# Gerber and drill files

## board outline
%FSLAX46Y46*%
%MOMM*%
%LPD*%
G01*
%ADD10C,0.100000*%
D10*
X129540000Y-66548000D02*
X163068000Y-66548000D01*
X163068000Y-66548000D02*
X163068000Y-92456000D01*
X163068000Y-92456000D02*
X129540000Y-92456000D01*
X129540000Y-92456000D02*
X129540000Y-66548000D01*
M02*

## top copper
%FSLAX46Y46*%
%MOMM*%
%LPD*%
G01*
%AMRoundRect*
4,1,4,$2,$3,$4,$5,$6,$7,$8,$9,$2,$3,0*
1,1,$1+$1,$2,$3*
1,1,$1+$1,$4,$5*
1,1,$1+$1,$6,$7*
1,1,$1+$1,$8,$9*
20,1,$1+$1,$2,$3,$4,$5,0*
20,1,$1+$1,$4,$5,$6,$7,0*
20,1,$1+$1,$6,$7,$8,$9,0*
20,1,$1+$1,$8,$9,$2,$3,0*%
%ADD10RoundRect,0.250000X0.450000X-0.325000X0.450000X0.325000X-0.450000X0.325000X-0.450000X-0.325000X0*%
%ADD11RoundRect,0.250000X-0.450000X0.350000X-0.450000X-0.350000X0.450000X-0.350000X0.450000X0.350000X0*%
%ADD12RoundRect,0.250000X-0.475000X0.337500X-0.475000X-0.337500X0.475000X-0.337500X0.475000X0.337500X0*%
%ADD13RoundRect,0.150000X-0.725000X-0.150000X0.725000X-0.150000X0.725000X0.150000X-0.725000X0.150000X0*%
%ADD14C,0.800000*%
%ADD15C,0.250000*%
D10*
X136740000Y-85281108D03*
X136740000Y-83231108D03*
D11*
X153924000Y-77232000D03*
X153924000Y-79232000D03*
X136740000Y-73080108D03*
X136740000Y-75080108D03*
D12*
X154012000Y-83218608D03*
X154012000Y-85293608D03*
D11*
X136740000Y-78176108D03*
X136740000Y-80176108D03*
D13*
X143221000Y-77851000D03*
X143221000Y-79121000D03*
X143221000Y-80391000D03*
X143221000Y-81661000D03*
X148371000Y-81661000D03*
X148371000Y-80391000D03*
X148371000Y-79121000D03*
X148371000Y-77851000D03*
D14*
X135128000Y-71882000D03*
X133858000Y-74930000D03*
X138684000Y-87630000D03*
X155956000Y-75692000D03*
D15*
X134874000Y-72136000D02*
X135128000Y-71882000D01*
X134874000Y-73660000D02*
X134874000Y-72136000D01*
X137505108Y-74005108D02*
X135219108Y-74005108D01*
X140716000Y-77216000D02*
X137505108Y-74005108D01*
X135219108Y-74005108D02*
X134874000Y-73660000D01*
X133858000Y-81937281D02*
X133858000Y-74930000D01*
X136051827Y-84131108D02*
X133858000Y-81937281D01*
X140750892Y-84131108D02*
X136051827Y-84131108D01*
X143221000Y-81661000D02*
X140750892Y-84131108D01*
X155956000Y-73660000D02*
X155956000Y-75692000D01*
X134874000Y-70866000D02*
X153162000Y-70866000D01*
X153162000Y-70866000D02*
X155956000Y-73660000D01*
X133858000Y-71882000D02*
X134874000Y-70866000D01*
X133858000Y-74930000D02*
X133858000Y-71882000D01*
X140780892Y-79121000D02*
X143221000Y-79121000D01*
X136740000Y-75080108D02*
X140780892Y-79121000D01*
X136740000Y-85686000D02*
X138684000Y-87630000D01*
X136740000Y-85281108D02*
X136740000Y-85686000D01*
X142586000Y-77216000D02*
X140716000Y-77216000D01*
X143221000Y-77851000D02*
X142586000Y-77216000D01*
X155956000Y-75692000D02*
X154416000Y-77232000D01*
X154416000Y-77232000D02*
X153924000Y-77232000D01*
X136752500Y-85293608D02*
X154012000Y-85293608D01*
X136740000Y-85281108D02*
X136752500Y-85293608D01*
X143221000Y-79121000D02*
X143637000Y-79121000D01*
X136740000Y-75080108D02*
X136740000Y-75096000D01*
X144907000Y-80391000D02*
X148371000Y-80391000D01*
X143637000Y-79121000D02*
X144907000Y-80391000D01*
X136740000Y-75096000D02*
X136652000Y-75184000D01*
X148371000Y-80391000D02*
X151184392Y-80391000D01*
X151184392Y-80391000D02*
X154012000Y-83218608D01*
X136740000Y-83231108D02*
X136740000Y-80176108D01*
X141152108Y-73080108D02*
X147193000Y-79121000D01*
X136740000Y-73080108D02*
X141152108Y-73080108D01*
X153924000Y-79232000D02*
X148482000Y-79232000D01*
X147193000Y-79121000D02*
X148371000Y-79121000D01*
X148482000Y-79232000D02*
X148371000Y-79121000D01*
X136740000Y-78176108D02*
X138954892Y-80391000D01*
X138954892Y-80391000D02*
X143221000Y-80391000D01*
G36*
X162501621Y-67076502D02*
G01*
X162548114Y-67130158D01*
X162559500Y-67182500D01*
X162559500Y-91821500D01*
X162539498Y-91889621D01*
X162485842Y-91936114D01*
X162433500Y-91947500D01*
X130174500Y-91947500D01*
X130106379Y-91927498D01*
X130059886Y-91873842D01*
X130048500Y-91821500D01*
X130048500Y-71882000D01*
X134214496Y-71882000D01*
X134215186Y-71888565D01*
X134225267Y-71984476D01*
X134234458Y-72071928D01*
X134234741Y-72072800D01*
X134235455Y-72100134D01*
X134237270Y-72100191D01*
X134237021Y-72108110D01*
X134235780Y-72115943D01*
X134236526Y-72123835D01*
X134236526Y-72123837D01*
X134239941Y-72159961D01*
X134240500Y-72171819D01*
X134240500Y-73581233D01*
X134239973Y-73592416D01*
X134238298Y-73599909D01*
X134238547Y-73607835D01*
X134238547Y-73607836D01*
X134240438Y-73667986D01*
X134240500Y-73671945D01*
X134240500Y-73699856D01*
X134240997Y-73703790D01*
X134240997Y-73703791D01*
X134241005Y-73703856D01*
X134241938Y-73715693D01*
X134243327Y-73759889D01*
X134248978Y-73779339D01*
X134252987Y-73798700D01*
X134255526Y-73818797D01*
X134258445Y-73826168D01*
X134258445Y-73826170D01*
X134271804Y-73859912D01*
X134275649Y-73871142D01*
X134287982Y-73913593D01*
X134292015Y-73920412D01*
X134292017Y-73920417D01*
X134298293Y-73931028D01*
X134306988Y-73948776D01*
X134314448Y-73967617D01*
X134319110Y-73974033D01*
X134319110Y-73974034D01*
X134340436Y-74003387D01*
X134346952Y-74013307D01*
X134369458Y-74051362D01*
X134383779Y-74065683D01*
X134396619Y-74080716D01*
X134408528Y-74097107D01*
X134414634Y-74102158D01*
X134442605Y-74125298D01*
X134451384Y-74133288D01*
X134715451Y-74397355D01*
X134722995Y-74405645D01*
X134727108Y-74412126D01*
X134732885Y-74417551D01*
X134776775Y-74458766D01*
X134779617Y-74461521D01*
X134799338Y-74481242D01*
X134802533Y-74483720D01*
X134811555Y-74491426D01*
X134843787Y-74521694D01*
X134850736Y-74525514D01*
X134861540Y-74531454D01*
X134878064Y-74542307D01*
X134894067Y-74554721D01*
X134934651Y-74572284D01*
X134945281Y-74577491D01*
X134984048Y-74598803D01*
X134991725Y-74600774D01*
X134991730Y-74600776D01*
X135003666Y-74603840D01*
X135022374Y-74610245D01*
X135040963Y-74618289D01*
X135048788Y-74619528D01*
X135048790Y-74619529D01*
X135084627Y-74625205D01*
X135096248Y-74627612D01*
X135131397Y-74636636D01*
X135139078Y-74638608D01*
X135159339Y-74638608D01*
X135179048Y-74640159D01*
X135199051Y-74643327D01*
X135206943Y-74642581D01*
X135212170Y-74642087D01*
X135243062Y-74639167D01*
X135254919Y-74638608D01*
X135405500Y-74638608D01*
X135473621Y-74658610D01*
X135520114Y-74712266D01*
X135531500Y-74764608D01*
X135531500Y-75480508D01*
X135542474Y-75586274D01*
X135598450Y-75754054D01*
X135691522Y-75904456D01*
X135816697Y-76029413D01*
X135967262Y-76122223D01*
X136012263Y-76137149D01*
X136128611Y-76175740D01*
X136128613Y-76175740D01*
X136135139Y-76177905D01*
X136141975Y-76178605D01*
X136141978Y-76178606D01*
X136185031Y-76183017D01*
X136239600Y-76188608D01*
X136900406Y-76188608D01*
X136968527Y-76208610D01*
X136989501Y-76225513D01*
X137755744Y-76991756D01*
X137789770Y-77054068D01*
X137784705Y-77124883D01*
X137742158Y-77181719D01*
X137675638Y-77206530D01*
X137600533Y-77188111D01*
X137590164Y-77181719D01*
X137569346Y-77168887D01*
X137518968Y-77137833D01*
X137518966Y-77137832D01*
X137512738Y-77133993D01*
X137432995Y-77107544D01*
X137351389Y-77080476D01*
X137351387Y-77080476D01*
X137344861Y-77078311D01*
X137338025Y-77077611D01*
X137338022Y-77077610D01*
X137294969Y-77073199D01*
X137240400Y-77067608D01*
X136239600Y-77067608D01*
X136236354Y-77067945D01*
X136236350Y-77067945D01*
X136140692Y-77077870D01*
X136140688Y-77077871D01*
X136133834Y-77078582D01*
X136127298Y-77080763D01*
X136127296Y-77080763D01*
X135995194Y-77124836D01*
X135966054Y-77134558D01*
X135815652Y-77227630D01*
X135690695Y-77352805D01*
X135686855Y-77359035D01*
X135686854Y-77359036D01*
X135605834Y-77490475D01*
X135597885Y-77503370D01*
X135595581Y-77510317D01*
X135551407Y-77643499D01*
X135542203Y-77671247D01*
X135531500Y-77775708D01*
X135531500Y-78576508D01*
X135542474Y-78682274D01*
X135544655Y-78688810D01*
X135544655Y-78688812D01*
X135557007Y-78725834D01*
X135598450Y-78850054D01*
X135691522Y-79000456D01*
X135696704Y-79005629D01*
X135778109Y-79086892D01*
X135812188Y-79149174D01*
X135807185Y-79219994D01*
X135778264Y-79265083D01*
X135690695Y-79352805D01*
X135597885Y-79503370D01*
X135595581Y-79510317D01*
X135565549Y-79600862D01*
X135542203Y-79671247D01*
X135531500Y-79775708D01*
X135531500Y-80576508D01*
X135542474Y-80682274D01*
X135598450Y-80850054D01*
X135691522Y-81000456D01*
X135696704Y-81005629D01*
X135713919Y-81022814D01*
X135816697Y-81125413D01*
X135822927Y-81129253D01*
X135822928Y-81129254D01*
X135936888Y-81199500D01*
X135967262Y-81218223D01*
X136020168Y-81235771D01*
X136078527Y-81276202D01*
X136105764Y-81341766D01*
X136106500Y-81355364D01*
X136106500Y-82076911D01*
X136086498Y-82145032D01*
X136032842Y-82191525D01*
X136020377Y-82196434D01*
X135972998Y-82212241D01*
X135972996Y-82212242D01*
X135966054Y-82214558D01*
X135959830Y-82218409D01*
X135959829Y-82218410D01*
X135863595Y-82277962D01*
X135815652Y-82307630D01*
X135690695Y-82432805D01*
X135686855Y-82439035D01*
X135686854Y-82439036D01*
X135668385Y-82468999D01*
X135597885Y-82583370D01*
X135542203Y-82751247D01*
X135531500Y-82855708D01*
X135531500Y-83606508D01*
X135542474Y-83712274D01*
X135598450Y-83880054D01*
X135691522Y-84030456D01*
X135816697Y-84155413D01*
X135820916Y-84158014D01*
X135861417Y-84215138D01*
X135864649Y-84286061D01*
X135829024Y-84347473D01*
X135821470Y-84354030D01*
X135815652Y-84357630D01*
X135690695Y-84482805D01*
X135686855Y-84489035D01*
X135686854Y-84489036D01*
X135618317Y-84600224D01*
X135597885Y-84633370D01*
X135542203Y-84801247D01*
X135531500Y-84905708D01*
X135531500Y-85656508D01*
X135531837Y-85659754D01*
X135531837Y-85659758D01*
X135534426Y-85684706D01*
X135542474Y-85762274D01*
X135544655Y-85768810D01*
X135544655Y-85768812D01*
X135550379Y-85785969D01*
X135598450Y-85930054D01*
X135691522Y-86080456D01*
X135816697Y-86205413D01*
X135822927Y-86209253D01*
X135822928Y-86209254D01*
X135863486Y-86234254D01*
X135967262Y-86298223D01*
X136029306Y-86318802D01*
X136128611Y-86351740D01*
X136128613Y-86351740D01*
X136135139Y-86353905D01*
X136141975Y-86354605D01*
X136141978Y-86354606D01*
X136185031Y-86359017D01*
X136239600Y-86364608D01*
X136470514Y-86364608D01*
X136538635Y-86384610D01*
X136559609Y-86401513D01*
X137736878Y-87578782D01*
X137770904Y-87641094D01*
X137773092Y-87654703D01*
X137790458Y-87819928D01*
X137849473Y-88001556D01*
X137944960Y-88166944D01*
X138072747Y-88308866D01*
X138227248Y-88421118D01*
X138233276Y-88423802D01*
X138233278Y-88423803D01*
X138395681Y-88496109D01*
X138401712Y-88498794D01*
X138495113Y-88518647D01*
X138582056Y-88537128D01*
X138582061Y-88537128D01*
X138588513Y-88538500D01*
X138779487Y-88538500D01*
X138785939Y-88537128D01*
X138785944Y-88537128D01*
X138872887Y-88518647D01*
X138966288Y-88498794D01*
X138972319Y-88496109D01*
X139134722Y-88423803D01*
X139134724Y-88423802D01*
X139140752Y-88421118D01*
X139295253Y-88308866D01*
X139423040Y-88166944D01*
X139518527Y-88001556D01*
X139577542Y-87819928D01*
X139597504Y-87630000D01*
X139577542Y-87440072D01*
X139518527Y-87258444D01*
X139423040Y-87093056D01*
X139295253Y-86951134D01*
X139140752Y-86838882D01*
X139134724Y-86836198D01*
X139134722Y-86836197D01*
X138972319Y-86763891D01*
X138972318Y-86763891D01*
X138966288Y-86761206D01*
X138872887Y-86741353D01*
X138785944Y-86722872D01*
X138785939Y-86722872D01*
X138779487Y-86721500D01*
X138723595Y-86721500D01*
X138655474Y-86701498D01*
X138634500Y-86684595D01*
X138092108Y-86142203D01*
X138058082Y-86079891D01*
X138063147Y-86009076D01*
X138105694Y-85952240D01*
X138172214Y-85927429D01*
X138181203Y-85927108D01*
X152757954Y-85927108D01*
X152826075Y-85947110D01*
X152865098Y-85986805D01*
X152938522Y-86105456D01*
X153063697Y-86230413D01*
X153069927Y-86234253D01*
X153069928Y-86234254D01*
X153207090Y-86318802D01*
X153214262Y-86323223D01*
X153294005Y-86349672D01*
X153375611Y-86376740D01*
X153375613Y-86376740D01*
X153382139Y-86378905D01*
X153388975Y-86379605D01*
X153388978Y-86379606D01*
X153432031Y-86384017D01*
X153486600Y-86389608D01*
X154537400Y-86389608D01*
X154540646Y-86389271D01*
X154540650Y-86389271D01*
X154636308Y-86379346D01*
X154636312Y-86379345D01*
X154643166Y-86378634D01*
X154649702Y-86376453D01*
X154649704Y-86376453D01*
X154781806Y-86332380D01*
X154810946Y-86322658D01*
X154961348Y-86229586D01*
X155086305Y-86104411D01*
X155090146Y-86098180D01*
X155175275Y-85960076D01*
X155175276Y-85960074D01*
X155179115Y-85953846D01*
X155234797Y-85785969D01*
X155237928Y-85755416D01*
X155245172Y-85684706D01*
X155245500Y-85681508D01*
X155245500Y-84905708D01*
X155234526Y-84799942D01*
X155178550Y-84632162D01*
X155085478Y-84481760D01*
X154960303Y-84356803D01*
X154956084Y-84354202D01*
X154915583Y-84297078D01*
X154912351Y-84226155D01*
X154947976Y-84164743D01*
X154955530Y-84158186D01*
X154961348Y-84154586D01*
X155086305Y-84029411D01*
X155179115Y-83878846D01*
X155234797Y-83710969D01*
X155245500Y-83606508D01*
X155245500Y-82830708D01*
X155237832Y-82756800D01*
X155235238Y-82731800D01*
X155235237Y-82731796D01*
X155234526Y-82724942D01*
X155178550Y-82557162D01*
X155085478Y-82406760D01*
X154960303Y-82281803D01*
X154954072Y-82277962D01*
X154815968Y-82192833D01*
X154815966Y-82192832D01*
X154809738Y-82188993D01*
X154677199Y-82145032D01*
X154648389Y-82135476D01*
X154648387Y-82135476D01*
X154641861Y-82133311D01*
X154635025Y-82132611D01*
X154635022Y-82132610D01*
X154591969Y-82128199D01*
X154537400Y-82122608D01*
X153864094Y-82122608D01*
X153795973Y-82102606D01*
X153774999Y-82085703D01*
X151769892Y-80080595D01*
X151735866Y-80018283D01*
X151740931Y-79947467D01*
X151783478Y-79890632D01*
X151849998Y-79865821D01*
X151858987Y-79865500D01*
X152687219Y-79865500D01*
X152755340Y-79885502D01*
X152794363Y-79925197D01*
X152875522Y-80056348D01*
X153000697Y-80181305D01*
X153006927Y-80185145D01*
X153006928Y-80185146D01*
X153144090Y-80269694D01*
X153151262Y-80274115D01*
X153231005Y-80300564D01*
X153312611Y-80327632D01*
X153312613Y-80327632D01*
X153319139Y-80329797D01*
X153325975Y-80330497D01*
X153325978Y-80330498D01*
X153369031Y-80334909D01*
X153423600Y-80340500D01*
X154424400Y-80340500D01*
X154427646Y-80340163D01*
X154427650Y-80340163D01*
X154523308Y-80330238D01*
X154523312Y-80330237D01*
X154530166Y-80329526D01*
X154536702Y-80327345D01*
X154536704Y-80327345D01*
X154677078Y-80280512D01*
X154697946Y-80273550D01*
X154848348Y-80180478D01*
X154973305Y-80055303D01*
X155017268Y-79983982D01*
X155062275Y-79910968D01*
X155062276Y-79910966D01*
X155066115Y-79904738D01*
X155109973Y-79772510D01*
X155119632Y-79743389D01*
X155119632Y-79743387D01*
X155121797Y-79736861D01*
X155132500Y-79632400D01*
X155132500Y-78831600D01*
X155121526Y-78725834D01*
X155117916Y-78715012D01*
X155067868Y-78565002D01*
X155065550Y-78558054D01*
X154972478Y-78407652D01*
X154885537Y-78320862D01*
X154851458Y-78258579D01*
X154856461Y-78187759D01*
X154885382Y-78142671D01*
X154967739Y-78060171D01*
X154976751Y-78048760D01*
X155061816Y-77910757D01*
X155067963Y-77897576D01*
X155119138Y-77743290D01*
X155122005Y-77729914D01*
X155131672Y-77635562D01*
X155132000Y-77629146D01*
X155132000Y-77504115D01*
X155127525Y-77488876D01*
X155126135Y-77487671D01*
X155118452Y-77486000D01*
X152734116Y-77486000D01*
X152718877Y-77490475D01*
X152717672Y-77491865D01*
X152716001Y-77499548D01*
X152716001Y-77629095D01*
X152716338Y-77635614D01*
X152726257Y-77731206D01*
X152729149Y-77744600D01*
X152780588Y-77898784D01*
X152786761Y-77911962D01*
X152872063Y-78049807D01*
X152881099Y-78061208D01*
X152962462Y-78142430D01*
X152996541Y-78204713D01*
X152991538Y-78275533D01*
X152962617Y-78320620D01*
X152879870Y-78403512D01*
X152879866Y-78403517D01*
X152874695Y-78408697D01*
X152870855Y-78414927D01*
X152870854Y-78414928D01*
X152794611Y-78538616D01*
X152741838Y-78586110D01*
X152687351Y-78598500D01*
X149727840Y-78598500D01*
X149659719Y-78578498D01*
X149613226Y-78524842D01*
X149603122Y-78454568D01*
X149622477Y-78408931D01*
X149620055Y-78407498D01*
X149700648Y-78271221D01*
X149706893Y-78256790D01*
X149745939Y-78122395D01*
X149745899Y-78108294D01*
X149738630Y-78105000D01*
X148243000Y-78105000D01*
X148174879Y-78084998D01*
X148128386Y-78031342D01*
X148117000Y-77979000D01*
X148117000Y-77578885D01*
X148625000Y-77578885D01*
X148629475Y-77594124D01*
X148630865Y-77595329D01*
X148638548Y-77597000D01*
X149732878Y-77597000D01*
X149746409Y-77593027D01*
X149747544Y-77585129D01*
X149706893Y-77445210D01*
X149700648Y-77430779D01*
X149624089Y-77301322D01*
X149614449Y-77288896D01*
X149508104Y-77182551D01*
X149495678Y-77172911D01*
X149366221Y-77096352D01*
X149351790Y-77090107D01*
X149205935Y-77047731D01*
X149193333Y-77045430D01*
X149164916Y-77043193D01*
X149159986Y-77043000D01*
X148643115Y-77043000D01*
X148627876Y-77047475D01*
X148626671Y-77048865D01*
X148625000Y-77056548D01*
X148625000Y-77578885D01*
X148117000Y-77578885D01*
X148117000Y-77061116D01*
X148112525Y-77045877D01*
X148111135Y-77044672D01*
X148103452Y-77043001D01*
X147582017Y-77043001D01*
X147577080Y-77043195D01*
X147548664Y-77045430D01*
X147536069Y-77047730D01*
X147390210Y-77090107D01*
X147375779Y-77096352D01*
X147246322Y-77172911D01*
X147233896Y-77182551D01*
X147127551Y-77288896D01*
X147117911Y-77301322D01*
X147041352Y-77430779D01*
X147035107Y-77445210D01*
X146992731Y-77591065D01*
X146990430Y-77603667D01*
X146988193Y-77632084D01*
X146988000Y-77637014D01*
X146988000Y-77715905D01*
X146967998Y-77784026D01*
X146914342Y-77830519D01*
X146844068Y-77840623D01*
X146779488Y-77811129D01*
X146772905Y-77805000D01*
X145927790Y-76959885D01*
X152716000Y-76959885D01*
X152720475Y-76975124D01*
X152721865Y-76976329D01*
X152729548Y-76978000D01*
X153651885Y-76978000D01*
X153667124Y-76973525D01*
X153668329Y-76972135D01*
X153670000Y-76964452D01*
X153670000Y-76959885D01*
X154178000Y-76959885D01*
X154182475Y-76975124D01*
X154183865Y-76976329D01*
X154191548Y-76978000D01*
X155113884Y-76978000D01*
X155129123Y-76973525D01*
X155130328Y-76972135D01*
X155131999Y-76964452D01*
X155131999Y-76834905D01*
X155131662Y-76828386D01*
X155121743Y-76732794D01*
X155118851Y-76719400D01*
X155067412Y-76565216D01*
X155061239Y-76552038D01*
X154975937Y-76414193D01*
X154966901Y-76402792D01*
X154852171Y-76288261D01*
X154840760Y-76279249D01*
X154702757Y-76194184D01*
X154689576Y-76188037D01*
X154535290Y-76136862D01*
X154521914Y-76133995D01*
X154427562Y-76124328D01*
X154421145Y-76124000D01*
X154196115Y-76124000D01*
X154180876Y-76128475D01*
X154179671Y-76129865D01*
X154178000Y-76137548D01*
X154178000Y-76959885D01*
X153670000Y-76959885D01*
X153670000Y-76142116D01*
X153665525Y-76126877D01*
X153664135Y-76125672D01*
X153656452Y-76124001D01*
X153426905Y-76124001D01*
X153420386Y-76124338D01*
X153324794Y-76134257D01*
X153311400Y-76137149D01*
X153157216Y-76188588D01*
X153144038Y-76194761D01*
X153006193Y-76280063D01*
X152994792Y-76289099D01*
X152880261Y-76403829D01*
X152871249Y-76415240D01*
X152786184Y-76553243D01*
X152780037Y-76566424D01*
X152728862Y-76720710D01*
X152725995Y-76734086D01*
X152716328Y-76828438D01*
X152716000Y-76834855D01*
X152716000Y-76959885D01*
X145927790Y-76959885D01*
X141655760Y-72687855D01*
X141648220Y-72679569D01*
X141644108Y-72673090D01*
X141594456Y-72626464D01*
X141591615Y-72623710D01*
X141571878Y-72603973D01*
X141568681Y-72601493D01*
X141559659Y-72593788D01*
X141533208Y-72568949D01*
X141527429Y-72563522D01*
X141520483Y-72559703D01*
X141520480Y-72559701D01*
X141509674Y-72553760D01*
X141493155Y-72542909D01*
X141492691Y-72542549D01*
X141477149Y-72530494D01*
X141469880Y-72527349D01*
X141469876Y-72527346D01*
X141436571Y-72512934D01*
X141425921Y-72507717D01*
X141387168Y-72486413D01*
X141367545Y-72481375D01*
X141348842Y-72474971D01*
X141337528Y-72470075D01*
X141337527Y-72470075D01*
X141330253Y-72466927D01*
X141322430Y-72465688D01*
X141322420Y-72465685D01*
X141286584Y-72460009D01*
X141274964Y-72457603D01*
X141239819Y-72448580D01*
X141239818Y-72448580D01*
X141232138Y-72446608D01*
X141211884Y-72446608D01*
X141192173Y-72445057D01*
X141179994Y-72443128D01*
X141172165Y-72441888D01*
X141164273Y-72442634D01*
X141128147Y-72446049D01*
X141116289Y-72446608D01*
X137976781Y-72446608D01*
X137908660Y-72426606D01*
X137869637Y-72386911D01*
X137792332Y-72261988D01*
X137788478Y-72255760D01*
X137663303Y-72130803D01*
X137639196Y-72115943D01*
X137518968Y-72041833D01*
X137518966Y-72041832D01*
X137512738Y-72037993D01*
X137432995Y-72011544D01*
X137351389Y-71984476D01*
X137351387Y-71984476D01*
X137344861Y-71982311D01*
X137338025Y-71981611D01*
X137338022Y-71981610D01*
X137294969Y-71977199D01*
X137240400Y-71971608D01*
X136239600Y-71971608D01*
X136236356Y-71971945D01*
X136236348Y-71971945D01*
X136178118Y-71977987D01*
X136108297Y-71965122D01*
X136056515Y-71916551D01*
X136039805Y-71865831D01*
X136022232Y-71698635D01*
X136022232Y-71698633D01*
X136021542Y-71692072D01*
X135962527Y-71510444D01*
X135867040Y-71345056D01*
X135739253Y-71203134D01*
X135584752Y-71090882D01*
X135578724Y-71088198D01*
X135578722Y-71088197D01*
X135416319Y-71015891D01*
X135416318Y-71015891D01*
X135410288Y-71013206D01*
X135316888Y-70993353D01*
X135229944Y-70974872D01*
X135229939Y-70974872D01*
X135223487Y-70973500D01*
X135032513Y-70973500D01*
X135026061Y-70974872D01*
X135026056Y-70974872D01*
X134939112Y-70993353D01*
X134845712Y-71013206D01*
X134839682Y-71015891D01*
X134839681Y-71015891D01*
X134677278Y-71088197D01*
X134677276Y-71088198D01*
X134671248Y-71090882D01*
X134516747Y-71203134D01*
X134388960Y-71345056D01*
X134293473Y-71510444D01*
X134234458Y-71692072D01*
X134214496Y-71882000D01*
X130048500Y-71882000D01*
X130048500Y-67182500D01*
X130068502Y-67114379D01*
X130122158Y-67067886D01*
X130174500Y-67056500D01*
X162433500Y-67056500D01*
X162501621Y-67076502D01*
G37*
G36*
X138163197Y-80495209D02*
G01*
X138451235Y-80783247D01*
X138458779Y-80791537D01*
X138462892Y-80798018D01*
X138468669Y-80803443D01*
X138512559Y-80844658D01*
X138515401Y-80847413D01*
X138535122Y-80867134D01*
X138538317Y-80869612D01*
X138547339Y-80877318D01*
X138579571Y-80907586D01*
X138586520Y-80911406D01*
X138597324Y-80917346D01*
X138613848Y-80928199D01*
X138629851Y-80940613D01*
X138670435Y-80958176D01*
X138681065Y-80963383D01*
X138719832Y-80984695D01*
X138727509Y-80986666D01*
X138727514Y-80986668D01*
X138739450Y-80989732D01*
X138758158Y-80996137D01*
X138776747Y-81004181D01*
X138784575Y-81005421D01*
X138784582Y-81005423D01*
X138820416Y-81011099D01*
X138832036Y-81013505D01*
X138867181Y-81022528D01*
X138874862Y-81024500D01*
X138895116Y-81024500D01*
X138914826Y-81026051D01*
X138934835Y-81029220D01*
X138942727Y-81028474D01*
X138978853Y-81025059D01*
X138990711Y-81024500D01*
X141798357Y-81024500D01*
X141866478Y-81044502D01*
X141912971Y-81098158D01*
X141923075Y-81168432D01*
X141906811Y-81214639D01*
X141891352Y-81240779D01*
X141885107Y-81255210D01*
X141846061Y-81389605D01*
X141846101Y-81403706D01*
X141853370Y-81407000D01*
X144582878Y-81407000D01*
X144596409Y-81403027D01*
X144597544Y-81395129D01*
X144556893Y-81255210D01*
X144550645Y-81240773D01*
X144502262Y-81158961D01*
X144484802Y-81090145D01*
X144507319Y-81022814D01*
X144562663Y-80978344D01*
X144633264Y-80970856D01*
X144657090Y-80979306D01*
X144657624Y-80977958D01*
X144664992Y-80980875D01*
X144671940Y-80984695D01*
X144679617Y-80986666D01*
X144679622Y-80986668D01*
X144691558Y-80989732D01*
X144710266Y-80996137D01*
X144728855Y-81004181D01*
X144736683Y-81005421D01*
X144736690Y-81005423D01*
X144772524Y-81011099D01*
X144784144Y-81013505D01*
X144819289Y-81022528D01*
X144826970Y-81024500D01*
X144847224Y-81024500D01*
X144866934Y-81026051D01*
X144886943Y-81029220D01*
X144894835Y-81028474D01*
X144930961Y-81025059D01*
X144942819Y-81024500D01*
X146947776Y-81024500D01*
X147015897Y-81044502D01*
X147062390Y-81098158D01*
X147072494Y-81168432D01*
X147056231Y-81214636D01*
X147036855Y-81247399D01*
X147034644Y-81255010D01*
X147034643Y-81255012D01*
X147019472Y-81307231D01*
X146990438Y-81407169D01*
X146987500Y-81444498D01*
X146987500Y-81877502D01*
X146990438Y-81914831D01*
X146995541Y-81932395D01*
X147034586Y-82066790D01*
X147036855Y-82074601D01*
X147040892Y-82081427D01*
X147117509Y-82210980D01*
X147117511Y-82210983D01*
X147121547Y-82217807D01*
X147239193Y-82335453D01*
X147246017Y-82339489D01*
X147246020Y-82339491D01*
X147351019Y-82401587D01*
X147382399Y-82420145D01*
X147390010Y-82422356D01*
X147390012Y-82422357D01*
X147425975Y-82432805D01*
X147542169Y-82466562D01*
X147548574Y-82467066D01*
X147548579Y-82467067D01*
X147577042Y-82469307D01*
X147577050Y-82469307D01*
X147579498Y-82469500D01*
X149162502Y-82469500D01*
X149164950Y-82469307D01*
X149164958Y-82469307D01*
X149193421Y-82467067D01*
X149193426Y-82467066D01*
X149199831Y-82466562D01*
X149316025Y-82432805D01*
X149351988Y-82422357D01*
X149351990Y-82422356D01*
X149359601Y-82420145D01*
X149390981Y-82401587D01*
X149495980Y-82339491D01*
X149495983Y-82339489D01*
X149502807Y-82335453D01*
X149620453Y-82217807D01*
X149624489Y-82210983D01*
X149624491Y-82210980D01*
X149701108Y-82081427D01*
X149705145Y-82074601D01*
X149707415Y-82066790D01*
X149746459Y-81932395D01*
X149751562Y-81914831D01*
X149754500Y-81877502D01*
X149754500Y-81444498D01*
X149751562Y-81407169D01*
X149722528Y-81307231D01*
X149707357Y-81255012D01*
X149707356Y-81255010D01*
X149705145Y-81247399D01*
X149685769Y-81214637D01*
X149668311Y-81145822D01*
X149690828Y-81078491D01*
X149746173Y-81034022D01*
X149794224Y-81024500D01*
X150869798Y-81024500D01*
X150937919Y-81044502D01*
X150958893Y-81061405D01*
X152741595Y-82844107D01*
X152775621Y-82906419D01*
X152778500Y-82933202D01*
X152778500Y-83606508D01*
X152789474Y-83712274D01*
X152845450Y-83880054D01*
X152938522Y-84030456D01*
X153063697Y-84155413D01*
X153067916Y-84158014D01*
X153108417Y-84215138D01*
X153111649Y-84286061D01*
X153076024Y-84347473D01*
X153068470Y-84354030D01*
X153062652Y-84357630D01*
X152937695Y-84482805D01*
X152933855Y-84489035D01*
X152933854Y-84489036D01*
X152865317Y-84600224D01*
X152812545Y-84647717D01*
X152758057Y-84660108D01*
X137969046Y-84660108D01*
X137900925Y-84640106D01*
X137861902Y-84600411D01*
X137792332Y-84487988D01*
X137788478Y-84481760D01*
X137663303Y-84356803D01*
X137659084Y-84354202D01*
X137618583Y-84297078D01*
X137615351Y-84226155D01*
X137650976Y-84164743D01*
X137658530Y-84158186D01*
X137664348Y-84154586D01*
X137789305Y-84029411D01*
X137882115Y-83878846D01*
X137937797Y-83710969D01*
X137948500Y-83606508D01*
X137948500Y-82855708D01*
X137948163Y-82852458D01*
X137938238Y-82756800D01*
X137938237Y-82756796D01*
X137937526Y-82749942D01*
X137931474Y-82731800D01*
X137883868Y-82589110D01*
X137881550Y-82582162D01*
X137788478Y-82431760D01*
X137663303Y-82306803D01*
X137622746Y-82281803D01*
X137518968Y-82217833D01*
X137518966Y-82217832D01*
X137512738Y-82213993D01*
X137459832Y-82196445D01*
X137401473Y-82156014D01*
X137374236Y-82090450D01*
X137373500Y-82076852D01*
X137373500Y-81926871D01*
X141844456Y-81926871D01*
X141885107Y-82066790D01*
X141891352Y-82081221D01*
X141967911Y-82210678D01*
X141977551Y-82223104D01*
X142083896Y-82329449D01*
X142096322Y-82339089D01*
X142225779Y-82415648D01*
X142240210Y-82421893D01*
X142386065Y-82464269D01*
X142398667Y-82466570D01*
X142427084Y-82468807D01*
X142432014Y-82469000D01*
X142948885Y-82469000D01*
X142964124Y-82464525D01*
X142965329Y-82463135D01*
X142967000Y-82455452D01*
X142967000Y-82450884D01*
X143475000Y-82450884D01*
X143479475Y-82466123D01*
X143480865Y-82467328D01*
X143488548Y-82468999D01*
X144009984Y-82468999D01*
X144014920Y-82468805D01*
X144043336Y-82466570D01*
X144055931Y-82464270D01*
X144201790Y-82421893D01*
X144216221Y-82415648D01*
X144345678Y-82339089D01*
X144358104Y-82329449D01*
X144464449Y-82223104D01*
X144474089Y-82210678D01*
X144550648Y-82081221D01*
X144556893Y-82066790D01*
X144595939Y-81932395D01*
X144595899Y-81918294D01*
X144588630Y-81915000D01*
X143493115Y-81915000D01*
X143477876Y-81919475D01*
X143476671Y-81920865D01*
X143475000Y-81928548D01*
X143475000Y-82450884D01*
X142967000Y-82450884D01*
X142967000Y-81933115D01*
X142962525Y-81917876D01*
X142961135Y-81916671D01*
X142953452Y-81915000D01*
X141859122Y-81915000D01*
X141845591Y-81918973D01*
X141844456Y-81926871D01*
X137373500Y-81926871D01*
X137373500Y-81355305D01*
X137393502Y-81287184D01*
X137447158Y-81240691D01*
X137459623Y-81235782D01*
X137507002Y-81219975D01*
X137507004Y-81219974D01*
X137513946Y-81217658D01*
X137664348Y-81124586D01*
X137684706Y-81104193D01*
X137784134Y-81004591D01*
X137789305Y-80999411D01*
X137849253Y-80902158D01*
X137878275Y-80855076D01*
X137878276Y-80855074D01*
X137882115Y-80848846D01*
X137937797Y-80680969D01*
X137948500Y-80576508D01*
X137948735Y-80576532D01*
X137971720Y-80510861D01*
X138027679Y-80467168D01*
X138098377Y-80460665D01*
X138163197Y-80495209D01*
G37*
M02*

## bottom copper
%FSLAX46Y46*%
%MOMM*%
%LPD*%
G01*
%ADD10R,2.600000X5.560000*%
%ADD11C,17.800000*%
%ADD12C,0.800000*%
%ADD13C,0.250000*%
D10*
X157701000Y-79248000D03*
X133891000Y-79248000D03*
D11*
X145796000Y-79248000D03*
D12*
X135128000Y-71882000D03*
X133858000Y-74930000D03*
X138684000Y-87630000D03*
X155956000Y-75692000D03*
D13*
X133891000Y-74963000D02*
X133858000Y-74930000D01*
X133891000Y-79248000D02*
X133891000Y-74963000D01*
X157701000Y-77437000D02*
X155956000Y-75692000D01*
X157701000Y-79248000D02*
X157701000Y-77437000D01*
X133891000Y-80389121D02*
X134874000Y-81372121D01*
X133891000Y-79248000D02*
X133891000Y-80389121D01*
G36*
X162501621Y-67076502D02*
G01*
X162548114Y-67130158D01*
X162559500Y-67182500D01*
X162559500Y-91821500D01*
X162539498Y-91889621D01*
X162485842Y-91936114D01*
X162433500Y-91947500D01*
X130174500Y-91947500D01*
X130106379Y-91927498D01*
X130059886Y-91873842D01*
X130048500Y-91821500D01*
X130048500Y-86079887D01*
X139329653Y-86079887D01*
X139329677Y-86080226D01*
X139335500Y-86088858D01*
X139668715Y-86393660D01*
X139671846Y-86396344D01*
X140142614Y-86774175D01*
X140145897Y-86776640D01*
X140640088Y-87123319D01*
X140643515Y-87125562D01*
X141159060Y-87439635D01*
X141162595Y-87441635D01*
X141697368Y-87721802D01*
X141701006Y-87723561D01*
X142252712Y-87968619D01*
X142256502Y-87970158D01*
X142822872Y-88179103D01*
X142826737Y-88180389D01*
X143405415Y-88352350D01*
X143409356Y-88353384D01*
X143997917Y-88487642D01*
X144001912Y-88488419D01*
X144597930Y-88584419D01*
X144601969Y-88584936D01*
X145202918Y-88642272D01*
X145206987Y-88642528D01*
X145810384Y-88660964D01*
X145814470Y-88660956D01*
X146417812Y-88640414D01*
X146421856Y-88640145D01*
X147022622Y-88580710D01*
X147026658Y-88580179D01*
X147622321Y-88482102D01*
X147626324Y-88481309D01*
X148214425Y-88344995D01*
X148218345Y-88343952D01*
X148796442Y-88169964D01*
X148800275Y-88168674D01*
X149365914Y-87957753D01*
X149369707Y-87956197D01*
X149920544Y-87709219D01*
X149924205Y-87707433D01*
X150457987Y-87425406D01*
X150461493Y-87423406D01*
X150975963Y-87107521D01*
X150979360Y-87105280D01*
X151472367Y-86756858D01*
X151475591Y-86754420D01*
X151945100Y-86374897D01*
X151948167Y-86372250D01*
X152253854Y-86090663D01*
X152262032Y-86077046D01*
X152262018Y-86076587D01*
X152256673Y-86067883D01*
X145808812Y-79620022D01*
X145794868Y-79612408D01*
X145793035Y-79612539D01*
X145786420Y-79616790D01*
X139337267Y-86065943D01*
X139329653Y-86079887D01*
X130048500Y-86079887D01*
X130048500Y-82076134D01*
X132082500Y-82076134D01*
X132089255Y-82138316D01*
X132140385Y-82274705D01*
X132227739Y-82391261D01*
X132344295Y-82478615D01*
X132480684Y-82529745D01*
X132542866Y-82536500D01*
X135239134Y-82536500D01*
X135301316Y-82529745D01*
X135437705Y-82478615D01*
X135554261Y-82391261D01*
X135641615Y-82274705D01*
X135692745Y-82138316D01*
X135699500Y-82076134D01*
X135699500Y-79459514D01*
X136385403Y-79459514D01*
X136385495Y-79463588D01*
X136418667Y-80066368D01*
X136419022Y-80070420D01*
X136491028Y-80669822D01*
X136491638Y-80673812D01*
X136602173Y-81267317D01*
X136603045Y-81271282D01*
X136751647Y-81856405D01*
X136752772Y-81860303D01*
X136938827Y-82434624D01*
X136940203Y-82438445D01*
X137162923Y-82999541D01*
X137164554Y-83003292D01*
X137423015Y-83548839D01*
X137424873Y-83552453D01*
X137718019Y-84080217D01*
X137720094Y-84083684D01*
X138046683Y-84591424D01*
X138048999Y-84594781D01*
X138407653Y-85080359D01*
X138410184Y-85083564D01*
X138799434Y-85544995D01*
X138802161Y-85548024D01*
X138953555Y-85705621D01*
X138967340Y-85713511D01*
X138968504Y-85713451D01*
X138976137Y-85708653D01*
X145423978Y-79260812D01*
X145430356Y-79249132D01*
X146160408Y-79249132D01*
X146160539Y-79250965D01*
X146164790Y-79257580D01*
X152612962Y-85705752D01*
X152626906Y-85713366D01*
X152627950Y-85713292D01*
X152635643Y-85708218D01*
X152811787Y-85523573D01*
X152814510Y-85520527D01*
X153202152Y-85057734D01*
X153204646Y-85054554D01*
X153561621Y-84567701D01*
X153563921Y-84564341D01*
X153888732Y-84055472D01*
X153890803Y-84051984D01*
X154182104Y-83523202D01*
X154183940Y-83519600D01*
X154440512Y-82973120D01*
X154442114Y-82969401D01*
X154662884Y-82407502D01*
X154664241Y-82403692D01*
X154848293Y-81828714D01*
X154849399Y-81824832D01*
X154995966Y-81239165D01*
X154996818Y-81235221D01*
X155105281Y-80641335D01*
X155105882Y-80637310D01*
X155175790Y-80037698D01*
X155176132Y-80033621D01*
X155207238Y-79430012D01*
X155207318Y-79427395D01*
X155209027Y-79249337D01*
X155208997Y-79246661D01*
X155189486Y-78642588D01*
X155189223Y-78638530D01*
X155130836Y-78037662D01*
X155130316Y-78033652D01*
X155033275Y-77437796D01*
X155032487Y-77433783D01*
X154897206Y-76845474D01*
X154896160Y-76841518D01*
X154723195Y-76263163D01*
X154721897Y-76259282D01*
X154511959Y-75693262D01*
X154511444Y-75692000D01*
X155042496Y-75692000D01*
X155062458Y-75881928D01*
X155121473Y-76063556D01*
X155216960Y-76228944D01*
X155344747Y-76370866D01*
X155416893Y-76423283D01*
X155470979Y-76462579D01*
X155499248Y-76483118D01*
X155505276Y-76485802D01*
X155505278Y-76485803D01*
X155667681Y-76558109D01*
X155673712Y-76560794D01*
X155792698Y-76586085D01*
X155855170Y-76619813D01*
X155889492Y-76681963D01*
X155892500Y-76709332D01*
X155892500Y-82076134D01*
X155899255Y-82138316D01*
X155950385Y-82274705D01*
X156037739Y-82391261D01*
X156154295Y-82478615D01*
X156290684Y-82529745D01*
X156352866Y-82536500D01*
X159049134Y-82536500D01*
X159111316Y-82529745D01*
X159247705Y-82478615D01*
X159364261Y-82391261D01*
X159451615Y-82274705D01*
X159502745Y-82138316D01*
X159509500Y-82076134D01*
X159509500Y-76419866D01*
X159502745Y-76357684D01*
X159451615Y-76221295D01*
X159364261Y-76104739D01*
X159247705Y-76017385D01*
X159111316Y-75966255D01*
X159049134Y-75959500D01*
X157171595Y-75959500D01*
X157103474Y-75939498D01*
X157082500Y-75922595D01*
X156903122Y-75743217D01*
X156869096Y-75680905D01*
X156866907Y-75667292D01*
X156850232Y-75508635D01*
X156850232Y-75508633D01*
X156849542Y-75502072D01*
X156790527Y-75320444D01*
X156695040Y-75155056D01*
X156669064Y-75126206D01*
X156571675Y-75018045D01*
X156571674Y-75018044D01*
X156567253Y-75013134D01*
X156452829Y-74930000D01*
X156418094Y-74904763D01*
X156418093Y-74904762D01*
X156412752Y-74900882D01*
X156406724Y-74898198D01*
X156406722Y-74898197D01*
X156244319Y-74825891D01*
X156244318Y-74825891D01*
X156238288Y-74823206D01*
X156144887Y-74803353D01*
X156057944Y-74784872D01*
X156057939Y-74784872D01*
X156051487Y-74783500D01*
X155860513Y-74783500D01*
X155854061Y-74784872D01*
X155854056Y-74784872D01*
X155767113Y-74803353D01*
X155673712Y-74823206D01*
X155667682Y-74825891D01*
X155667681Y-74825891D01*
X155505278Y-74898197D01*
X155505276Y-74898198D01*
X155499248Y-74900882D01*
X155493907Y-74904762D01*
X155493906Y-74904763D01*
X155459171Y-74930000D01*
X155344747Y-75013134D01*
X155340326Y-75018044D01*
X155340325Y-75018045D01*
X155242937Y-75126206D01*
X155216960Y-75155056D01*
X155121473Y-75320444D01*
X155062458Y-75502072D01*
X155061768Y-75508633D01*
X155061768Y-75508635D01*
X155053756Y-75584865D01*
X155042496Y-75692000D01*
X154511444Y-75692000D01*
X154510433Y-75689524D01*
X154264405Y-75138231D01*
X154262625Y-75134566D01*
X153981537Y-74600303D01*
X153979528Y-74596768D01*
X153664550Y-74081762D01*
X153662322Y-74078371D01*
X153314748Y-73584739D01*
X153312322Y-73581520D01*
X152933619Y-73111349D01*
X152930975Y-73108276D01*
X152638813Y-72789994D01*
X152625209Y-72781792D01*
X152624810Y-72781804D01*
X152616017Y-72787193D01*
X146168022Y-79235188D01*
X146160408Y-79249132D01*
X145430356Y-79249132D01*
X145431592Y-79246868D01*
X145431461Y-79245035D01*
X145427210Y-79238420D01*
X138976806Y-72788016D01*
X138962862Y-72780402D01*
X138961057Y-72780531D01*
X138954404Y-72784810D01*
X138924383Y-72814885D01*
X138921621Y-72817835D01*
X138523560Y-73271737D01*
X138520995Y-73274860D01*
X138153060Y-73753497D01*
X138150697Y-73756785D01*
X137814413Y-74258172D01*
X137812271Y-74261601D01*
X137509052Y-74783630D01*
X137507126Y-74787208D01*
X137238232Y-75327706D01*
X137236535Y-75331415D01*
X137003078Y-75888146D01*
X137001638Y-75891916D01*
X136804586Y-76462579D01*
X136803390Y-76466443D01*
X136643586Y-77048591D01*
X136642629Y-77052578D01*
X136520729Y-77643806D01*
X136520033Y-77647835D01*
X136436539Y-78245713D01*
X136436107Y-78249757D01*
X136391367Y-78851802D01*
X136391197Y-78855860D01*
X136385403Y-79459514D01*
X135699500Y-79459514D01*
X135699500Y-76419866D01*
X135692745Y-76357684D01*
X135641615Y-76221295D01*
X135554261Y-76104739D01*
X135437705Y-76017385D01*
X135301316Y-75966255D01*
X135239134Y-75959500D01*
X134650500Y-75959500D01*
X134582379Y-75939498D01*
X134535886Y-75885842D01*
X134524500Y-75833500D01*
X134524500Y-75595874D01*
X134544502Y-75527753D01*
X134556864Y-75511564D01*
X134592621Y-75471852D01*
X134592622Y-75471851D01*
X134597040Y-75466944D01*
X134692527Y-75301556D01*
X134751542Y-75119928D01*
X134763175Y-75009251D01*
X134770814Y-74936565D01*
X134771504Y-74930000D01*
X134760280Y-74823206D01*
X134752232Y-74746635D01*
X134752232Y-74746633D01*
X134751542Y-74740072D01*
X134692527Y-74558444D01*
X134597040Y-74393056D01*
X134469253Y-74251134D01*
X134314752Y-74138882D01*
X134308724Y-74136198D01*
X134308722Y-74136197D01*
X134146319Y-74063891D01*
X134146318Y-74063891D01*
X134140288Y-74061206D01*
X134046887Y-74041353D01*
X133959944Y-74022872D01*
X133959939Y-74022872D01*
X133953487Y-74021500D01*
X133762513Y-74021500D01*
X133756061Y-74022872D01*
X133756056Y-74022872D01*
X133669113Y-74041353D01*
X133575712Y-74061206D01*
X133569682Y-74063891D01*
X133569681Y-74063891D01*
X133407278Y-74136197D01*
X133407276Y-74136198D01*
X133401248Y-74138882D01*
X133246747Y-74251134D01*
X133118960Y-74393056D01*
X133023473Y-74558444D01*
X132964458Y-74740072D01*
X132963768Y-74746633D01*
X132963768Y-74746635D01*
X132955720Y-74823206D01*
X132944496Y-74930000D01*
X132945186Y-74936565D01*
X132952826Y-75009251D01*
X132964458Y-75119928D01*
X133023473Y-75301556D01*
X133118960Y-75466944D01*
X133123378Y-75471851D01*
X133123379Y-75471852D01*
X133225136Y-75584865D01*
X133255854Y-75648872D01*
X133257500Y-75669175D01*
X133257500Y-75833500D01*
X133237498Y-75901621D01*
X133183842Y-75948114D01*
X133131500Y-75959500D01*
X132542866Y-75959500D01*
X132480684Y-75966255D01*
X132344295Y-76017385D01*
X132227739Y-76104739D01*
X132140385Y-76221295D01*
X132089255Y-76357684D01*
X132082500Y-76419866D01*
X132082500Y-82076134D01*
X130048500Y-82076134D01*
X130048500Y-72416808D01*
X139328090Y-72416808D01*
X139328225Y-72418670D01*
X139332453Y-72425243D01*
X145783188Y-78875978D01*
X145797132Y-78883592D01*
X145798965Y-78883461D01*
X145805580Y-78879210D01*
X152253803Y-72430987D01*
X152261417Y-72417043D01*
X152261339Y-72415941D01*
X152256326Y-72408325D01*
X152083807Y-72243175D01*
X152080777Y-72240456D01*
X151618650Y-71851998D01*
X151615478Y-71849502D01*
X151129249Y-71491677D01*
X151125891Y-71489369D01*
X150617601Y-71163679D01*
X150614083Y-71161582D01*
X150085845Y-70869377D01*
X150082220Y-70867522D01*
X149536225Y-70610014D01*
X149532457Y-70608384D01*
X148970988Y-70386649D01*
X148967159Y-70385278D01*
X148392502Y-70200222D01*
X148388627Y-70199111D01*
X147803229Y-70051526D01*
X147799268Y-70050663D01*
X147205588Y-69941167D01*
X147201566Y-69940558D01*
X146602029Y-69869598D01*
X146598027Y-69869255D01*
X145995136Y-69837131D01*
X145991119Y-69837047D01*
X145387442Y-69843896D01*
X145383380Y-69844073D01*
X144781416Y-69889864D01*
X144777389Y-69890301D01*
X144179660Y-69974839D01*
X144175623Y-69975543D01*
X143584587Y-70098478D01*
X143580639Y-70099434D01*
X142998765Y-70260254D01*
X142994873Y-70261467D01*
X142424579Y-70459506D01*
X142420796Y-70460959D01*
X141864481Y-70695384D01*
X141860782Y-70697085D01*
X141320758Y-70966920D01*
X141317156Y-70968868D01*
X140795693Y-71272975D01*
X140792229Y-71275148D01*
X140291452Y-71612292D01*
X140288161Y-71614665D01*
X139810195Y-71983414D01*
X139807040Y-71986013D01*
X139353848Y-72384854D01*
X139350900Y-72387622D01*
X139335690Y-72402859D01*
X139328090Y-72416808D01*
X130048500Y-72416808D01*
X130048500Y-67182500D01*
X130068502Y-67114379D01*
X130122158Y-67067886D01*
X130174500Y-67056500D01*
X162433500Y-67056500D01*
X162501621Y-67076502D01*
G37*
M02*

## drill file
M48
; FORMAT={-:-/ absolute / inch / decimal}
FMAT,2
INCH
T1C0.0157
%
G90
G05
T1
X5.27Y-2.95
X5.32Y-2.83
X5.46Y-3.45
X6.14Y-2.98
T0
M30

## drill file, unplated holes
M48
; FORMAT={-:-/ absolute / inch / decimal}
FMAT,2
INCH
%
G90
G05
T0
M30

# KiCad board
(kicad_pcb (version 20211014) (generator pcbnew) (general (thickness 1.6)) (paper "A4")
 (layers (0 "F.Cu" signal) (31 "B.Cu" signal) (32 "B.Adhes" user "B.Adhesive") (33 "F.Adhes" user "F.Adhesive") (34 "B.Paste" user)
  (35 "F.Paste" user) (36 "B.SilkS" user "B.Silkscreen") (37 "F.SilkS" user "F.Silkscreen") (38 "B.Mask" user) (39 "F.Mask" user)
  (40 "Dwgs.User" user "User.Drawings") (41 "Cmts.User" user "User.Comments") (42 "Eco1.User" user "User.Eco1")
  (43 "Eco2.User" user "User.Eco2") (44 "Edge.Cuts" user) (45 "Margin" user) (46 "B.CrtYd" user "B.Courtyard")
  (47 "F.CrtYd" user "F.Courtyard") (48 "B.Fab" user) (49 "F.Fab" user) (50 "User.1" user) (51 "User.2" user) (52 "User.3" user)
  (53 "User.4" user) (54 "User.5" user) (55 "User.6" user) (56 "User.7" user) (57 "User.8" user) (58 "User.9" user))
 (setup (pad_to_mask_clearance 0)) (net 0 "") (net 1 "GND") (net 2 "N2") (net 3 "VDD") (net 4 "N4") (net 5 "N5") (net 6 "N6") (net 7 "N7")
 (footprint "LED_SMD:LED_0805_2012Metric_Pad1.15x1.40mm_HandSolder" (layer "F.Cu") (at 136.74 84.256108 90)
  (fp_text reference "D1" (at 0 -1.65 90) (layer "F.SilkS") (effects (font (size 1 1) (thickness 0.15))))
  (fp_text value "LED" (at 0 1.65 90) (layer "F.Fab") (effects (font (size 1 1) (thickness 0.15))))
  (pad "1" smd roundrect (at -1.025 0 90) (size 1.15 1.4) (layers "F.Cu" "F.Paste" "F.Mask") (roundrect_rratio 0.2173913043) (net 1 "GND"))
  (pad "2" smd roundrect (at 1.025 0 90) (size 1.15 1.4) (layers "F.Cu" "F.Paste" "F.Mask") (roundrect_rratio 0.2173913043) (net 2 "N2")))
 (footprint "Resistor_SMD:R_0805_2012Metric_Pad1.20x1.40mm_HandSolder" (layer "F.Cu") (at 153.924 78.232 -90)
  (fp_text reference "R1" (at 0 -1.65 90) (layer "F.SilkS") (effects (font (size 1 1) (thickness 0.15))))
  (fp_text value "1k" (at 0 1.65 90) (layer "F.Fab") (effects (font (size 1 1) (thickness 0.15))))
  (pad "1" smd roundrect (at -1 0 270) (size 1.2 1.4) (layers "F.Cu" "F.Paste" "F.Mask") (roundrect_rratio 0.2083333333) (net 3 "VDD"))
  (pad "2" smd roundrect (at 1 0 270) (size 1.2 1.4) (layers "F.Cu" "F.Paste" "F.Mask") (roundrect_rratio 0.2083333333) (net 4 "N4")))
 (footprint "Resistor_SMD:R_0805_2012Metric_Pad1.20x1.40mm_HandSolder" (layer "F.Cu") (at 136.74 74.080108 -90)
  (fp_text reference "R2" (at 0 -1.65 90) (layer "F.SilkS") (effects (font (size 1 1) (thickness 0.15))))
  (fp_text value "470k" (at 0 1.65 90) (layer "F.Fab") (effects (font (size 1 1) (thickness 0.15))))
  (pad "1" smd roundrect (at -1 0 270) (size 1.2 1.4) (layers "F.Cu" "F.Paste" "F.Mask") (roundrect_rratio 0.2083333333) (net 4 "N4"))
  (pad "2" smd roundrect (at 1 0 270) (size 1.2 1.4) (layers "F.Cu" "F.Paste" "F.Mask") (roundrect_rratio 0.2083333333) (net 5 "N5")))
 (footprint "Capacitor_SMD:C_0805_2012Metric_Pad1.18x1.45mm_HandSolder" (layer "F.Cu") (at 154.012 84.256108 -90)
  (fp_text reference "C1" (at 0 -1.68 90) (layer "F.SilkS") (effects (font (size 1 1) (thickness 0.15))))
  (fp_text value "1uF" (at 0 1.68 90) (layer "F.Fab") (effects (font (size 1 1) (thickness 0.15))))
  (pad "1" smd roundrect (at -1.0375 0 270) (size 1.175 1.45) (layers "F.Cu" "F.Paste" "F.Mask") (roundrect_rratio 0.2127659574)
   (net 5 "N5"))
  (pad "2" smd roundrect (at 1.0375 0 270) (size 1.175 1.45) (layers "F.Cu" "F.Paste" "F.Mask") (roundrect_rratio 0.2127659574)
   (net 1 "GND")))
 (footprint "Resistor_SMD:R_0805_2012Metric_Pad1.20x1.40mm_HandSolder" (layer "F.Cu") (at 136.74 79.176108 -90)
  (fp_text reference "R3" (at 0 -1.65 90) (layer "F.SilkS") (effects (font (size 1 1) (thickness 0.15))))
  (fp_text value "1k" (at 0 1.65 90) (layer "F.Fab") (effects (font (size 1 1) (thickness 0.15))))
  (pad "1" smd roundrect (at -1 0 270) (size 1.2 1.4) (layers "F.Cu" "F.Paste" "F.Mask") (roundrect_rratio 0.2083333333) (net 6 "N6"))
  (pad "2" smd roundrect (at 1 0 270) (size 1.2 1.4) (layers "F.Cu" "F.Paste" "F.Mask") (roundrect_rratio 0.2083333333) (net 2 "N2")))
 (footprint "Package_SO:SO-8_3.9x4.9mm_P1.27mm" (layer "F.Cu") (at 145.796 79.756)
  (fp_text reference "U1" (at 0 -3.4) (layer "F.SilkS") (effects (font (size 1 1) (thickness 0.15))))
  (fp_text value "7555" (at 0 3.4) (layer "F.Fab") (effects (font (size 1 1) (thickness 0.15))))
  (pad "1" smd roundrect (at -2.575 -1.905) (size 1.75 0.6) (layers "F.Cu" "F.Paste" "F.Mask") (roundrect_rratio 0.25) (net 1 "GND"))
  (pad "2" smd roundrect (at -2.575 -0.635) (size 1.75 0.6) (layers "F.Cu" "F.Paste" "F.Mask") (roundrect_rratio 0.25) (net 5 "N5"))
  (pad "3" smd roundrect (at -2.575 0.635) (size 1.75 0.6) (layers "F.Cu" "F.Paste" "F.Mask") (roundrect_rratio 0.25) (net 6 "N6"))
  (pad "4" smd roundrect (at -2.575 1.905) (size 1.75 0.6) (layers "F.Cu" "F.Paste" "F.Mask") (roundrect_rratio 0.25) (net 3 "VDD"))
  (pad "5" smd roundrect (at 2.575 1.905) (size 1.75 0.6) (layers "F.Cu" "F.Paste" "F.Mask") (roundrect_rratio 0.25) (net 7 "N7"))
  (pad "6" smd roundrect (at 2.575 0.635) (size 1.75 0.6) (layers "F.Cu" "F.Paste" "F.Mask") (roundrect_rratio 0.25) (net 5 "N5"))
  (pad "7" smd roundrect (at 2.575 -0.635) (size 1.75 0.6) (layers "F.Cu" "F.Paste" "F.Mask") (roundrect_rratio 0.25) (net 4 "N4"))
  (pad "8" smd roundrect (at 2.575 -1.905) (size 1.75 0.6) (layers "F.Cu" "F.Paste" "F.Mask") (roundrect_rratio 0.25) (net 3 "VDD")))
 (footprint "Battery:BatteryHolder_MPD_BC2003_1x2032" (layer "B.Cu") (at 145.796 79.248 180)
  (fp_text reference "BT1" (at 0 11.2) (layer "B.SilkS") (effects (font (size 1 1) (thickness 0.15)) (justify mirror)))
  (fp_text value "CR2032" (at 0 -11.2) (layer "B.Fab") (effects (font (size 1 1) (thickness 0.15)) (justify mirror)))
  (pad "1" smd rect (at -11.905 0 180) (size 2.6 5.56) (layers "B.Cu" "B.Paste" "B.Mask") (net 3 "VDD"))
  (pad "1" smd rect (at 11.905 0 180) (size 2.6 5.56) (layers "B.Cu" "B.Paste" "B.Mask") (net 3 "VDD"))
  (pad "2" smd circle (at 0 0 180) (size 17.8 17.8) (layers "B.Cu" "B.Mask") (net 1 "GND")))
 (gr_rect (start 129.54 66.548) (end 163.068 92.456) (layer "Edge.Cuts") (width 0.1) (fill none))
 (segment (start 143.221 81.661) (end 140.750892 84.131108) (width 0.25) (layer "F.Cu") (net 3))
 (segment (start 133.858 81.937281) (end 133.858 74.93) (width 0.25) (layer "F.Cu") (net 3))
 (segment (start 140.750892 84.131108) (end 136.051827 84.131108) (width 0.25) (layer "F.Cu") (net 3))
 (segment (start 154.416 77.232) (end 153.924 77.232) (width 0.25) (layer "F.Cu") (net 3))
 (segment (start 153.162 70.866) (end 155.956 73.66) (width 0.25) (layer "F.Cu") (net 3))
 (segment (start 155.956 75.692) (end 154.416 77.232) (width 0.25) (layer "F.Cu") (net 3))
 (segment (start 133.858 74.93) (end 133.858 71.882) (width 0.25) (layer "F.Cu") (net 3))
 (segment (start 133.858 71.882) (end 134.874 70.866) (width 0.25) (layer "F.Cu") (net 3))
 (segment (start 136.051827 84.131108) (end 133.858 81.937281) (width 0.25) (layer "F.Cu") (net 3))
 (segment (start 134.874 70.866) (end 153.162 70.866) (width 0.25) (layer "F.Cu") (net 3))
 (segment (start 155.956 73.66) (end 155.956 75.692) (width 0.25) (layer "F.Cu") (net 3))
 (via (at 155.956 75.692) (size 0.8) (drill 0.4) (layers "F.Cu" "B.Cu") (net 3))
 (via (at 133.858 74.93) (size 0.8) (drill 0.4) (layers "F.Cu" "B.Cu") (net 3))
 (segment (start 133.891 79.248) (end 133.891 74.963) (width 0.25) (layer "B.Cu") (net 3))
 (segment (start 133.891 80.389121) (end 134.874 81.372121) (width 0.25) (layer "B.Cu") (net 3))
 (segment (start 133.891 74.963) (end 133.858 74.93) (width 0.25) (layer "B.Cu") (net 3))
 (segment (start 157.701 77.437) (end 155.956 75.692) (width 0.25) (layer "B.Cu") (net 3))
 (segment (start 133.891 79.248) (end 133.891 80.389121) (width 0.25) (layer "B.Cu") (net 3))
 (segment (start 157.701 79.248) (end 157.701 77.437) (width 0.25) (layer "B.Cu") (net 3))
 (segment (start 136.7525 85.293608) (end 154.012 85.293608) (width 0.25) (layer "F.Cu") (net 1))
 (segment (start 135.219108 74.005108) (end 134.874 73.66) (width 0.25) (layer "F.Cu") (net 1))
 (segment (start 134.874 72.136) (end 135.128 71.882) (width 0.25) (layer "F.Cu") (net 1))
 (segment (start 137.505108 74.005108) (end 135.219108 74.005108) (width 0.25) (layer "F.Cu") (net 1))
 (segment (start 136.74 85.686) (end 138.684 87.63) (width 0.25) (layer "F.Cu") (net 1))
 (segment (start 136.74 85.281108) (end 136.7525 85.293608) (width 0.25) (layer "F.Cu") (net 1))
 (segment (start 140.716 77.216) (end 137.505108 74.005108) (width 0.25) (layer "F.Cu") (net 1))
 (segment (start 136.74 85.281108) (end 136.74 85.686) (width 0.25) (layer "F.Cu") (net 1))
 (segment (start 143.221 77.851) (end 142.586 77.216) (width 0.25) (layer "F.Cu") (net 1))
 (segment (start 134.874 73.66) (end 134.874 72.136) (width 0.25) (layer "F.Cu") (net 1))
 (segment (start 142.586 77.216) (end 140.716 77.216) (width 0.25) (layer "F.Cu") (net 1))
 (via (at 135.128 71.882) (size 0.8) (drill 0.4) (layers "F.Cu" "B.Cu") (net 1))
 (via (at 138.684 87.63) (size 0.8) (drill 0.4) (layers "F.Cu" "B.Cu") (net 1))
 (segment (start 143.221 79.121) (end 143.637 79.121) (width 0.25) (layer "F.Cu") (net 5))
 (segment (start 136.74 75.080108) (end 136.74 75.096) (width 0.25) (layer "F.Cu") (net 5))
 (segment (start 144.907 80.391) (end 148.371 80.391) (width 0.25) (layer "F.Cu") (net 5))
 (segment (start 140.780892 79.121) (end 143.221 79.121) (width 0.25) (layer "F.Cu") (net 5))
 (segment (start 143.637 79.121) (end 144.907 80.391) (width 0.25) (layer "F.Cu") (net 5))
 (segment (start 136.74 75.096) (end 136.652 75.184) (width 0.25) (layer "F.Cu") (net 5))
 (segment (start 136.74 75.080108) (end 140.780892 79.121) (width 0.25) (layer "F.Cu") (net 5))
 (segment (start 148.371 80.391) (end 151.184392 80.391) (width 0.25) (layer "F.Cu") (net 5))
 (segment (start 151.184392 80.391) (end 154.012 83.218608) (width 0.25) (layer "F.Cu") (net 5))
 (segment (start 136.74 83.231108) (end 136.74 80.176108) (width 0.25) (layer "F.Cu") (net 2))
 (segment (start 141.152108 73.080108) (end 147.193 79.121) (width 0.25) (layer "F.Cu") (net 4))
 (segment (start 136.74 73.080108) (end 141.152108 73.080108) (width 0.25) (layer "F.Cu") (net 4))
 (segment (start 153.924 79.232) (end 148.482 79.232) (width 0.25) (layer "F.Cu") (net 4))
 (segment (start 147.193 79.121) (end 148.371 79.121) (width 0.25) (layer "F.Cu") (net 4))
 (segment (start 148.482 79.232) (end 148.371 79.121) (width 0.25) (layer "F.Cu") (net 4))
 (segment (start 136.74 78.176108) (end 138.954892 80.391) (width 0.25) (layer "F.Cu") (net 6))
 (segment (start 138.954892 80.391) (end 143.221 80.391) (width 0.25) (layer "F.Cu") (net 6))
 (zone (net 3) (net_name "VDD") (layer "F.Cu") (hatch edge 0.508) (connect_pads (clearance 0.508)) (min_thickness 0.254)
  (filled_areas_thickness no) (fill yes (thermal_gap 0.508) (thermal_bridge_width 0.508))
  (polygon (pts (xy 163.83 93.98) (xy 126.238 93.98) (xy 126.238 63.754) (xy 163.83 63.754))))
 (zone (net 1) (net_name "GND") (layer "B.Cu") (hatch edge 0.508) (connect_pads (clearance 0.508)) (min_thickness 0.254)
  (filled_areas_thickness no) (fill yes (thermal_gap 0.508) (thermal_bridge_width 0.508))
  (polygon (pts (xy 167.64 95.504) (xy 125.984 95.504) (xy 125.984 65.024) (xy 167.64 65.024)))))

